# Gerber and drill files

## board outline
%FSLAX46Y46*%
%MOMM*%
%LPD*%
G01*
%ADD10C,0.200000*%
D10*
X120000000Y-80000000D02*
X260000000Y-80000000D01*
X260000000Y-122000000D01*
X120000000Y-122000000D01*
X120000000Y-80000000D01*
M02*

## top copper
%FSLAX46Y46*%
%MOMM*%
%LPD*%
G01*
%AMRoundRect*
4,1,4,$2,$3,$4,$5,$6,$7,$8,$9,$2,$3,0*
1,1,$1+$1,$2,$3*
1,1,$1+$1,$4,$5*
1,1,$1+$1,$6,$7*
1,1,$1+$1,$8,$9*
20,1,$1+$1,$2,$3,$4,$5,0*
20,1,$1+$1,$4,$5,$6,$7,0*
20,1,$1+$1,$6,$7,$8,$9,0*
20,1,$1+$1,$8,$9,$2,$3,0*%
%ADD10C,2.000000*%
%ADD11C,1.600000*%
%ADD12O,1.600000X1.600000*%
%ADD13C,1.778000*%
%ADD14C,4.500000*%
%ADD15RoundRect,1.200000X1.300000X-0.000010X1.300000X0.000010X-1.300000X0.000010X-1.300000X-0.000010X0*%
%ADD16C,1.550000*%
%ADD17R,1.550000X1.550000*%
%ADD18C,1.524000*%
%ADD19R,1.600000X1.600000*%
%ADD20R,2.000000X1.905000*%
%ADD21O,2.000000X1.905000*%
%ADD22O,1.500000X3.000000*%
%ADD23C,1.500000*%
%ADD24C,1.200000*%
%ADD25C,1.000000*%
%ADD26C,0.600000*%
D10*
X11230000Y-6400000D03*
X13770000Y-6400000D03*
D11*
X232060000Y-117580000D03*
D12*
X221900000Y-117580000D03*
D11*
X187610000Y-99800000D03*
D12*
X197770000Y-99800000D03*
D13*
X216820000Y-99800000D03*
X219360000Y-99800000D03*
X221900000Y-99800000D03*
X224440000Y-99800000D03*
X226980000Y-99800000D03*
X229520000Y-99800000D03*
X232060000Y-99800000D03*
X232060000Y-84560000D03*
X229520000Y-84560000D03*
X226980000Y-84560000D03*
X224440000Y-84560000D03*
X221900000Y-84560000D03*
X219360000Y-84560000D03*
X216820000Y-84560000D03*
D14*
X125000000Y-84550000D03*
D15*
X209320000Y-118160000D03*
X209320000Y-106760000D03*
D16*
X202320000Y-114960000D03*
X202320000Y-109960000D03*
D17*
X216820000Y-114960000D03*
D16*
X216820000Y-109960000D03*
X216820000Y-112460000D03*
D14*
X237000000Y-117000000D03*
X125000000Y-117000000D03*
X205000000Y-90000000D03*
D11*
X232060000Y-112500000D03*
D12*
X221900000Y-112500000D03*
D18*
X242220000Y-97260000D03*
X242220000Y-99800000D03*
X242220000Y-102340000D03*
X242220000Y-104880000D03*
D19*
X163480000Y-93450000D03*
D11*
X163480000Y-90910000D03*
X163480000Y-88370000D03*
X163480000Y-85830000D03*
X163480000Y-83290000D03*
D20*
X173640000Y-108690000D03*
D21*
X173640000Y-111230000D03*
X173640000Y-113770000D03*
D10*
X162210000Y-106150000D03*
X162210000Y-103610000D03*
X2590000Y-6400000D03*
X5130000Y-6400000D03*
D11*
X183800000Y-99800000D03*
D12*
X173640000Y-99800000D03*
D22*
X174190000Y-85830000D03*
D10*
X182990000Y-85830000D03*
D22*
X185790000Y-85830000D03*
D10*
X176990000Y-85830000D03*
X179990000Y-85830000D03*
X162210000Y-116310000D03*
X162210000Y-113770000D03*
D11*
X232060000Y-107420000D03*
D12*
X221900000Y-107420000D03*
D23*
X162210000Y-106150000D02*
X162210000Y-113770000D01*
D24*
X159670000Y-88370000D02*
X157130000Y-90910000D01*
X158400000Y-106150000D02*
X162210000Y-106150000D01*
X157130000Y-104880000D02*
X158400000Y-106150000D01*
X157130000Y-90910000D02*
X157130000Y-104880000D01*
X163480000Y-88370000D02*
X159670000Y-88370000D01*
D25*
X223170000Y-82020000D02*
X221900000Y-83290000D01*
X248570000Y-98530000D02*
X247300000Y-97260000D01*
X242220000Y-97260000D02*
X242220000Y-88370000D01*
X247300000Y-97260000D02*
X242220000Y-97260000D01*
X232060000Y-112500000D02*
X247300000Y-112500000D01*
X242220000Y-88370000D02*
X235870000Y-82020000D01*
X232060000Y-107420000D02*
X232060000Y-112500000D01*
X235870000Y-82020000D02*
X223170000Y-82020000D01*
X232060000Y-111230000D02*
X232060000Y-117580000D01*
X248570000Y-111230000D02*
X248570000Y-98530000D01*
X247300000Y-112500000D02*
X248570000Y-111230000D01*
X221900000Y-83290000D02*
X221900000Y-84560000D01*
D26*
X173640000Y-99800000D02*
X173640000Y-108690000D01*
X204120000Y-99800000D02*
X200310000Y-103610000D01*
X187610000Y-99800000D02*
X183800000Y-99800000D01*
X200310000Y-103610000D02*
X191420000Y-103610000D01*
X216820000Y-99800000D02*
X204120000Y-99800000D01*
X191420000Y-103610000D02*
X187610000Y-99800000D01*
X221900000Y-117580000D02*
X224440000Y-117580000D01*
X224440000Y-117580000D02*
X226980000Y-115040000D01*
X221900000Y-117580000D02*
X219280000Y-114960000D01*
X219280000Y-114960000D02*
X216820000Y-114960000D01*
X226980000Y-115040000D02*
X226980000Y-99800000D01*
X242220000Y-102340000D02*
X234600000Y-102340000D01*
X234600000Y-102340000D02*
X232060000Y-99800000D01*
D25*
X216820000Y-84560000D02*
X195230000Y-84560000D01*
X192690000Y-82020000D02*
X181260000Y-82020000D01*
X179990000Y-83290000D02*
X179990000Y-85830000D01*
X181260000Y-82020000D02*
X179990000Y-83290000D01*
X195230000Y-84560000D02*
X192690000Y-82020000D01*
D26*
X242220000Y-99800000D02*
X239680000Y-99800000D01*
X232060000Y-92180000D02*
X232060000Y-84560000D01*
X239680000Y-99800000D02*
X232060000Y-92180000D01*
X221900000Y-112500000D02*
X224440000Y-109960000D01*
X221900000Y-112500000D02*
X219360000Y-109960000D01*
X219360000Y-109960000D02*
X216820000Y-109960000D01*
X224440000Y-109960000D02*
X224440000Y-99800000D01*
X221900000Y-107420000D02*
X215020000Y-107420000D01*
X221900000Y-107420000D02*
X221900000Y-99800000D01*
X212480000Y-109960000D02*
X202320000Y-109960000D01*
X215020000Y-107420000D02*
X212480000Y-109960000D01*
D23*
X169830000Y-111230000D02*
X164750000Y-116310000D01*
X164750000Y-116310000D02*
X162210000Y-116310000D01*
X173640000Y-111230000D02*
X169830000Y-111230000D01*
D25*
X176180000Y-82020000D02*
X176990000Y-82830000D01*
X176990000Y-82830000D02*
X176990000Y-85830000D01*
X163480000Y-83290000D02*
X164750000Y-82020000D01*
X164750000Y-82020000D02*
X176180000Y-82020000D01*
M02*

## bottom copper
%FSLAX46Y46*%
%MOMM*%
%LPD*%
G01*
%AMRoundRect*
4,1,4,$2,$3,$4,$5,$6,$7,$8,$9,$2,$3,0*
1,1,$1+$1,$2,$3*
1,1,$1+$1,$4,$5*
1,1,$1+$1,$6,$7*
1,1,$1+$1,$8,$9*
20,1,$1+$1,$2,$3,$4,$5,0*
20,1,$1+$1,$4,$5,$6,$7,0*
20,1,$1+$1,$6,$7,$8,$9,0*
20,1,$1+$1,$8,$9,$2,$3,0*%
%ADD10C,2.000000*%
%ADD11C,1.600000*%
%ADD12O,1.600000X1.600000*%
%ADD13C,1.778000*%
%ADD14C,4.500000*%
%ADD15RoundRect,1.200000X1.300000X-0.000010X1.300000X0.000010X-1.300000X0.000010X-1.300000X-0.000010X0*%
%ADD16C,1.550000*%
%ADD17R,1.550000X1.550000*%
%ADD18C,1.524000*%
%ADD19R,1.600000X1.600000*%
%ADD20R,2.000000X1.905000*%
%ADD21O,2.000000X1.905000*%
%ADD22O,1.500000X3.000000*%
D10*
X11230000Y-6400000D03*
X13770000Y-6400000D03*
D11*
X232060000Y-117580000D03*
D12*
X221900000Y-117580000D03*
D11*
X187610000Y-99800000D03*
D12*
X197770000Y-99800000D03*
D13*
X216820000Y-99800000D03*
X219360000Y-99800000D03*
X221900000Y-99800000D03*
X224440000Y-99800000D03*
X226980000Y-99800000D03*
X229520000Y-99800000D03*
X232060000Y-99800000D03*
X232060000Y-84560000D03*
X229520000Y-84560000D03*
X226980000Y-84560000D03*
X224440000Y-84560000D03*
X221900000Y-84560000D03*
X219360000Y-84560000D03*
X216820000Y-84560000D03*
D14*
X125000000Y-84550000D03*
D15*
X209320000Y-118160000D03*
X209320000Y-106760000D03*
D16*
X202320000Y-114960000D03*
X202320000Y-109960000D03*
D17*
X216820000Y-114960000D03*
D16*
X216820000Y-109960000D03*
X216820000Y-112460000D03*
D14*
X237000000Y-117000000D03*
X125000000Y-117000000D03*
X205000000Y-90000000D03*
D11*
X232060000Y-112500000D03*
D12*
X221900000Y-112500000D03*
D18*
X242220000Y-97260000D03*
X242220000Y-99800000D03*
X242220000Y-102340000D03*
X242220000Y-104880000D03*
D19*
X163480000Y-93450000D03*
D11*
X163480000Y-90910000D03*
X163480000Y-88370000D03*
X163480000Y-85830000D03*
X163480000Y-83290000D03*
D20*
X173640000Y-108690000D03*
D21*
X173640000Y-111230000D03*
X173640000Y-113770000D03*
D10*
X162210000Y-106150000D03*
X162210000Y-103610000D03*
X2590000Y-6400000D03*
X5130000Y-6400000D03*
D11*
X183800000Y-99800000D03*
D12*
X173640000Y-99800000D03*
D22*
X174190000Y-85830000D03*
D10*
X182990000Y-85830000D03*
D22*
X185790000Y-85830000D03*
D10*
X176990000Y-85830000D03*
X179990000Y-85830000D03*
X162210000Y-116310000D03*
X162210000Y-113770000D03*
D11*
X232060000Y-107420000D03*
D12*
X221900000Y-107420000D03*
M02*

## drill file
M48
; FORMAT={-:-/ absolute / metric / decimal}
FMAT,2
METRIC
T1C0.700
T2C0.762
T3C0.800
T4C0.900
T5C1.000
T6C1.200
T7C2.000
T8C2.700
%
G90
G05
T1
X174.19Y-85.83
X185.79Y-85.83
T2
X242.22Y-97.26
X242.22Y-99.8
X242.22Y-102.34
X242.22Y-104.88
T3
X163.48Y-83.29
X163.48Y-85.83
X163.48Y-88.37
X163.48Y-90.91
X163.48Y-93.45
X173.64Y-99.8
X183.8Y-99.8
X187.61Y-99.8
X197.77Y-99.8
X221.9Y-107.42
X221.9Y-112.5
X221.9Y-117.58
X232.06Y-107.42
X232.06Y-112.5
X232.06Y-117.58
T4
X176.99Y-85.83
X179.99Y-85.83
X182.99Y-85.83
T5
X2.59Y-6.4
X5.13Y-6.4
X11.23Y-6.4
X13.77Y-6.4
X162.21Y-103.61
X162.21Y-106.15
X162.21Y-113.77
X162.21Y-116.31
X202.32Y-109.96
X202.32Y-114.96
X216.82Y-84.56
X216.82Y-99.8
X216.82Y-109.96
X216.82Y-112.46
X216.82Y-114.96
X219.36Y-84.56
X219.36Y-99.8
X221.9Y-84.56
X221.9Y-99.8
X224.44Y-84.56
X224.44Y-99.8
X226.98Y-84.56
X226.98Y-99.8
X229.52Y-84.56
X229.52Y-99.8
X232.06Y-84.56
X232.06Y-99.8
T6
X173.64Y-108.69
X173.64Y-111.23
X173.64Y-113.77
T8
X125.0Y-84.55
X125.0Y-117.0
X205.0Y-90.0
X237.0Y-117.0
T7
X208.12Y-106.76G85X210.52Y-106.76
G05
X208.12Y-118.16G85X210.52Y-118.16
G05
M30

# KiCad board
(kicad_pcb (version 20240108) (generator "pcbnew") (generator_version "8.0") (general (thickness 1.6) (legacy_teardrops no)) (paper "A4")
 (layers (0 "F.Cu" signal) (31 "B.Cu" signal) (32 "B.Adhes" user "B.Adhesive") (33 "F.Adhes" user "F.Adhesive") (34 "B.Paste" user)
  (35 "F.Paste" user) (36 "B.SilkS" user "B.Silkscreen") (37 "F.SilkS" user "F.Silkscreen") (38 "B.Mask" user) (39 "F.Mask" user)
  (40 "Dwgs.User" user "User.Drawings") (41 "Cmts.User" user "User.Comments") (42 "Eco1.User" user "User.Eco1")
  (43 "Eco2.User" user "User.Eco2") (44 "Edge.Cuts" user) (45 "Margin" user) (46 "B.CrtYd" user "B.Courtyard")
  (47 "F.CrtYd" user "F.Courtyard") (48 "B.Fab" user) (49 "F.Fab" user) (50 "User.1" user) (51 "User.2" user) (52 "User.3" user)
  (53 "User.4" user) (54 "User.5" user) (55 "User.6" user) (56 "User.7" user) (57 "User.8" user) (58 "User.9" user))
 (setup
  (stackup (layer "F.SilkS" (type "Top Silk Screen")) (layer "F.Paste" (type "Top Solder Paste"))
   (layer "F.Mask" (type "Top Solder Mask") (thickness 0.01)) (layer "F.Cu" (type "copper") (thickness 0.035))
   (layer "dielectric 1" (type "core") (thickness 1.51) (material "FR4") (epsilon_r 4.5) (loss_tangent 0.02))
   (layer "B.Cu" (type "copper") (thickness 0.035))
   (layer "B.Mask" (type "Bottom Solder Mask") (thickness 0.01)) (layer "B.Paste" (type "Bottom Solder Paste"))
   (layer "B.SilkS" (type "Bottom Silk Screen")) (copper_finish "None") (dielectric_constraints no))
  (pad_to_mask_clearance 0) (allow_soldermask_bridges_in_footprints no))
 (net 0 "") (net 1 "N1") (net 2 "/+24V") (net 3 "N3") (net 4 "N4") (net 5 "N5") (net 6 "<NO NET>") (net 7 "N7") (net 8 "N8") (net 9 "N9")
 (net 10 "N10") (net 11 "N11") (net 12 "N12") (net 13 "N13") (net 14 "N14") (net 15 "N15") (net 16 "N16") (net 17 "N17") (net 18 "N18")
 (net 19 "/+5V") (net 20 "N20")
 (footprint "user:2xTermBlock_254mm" (layer "F.Cu") (at 11.23 6.4)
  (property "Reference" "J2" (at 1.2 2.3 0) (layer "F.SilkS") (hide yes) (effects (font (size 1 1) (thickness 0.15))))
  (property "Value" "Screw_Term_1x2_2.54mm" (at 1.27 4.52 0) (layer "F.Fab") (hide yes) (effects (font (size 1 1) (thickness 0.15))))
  (pad "1" thru_hole circle (at 0 0) (size 2 2) (drill 1) (layers "*.Cu" "*.Mask") (remove_unused_layers no) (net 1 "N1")
   (thermal_bridge_angle 90))
  (pad "2" thru_hole circle (at 2.54 0) (size 2 2) (drill 1) (layers "*.Cu" "*.Mask") (remove_unused_layers no) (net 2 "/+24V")))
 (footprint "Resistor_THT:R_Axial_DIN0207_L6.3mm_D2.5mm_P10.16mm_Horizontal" (layer "F.Cu") (at 232.06 117.58 180)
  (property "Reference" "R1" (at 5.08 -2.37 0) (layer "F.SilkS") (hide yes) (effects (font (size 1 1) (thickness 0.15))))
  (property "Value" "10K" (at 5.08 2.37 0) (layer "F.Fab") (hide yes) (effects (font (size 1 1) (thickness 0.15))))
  (pad "1" thru_hole circle (at 0 0 180) (size 1.6 1.6) (drill 0.8) (layers "*.Cu" "*.Mask") (remove_unused_layers no) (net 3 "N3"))
  (pad "2" thru_hole oval (at 10.16 0 180) (size 1.6 1.6) (drill 0.8) (layers "*.Cu" "*.Mask") (remove_unused_layers no) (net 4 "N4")))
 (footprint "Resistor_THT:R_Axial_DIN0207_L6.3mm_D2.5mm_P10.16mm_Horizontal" (layer "F.Cu") (at 187.61 99.8)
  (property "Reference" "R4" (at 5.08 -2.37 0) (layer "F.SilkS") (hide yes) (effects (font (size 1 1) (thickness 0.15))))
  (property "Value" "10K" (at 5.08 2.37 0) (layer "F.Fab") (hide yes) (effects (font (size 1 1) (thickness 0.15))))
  (pad "1" thru_hole circle (at 0 0) (size 1.6 1.6) (drill 0.8) (layers "*.Cu" "*.Mask") (remove_unused_layers no) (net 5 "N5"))
  (pad "2" thru_hole oval (at 10.16 0) (size 1.6 1.6) (drill 0.8) (layers "*.Cu" "*.Mask") (remove_unused_layers no) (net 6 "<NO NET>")))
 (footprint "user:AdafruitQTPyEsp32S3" (layer "F.Cu") (at 216.82 99.8 90)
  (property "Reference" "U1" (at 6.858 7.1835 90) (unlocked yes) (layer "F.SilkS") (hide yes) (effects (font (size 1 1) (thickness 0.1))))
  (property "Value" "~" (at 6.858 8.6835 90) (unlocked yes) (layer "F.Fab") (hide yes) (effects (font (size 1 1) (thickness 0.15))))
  (pad "1" thru_hole circle (at 0 0 90) (size 1.778 1.778) (drill 1) (layers "*.Cu" "*.Mask") (remove_unused_layers no) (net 5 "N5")
   (solder_mask_margin 0.0508) (thermal_bridge_angle 0))
  (pad "2" thru_hole circle (at 0 2.54 90) (size 1.778 1.778) (drill 1) (layers "*.Cu" "*.Mask") (remove_unused_layers no) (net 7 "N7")
   (solder_mask_margin 0.0508) (thermal_bridge_angle 0))
  (pad "3" thru_hole circle (at 0 5.08 90) (size 1.778 1.778) (drill 1) (layers "*.Cu" "*.Mask") (remove_unused_layers no) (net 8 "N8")
   (solder_mask_margin 0.0508) (thermal_bridge_angle 0))
  (pad "4" thru_hole circle (at 0 7.62 90) (size 1.778 1.778) (drill 1) (layers "*.Cu" "*.Mask") (remove_unused_layers no) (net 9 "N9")
   (solder_mask_margin 0.0508) (thermal_bridge_angle 0))
  (pad "5" thru_hole circle (at 0 10.16 90) (size 1.778 1.778) (drill 1) (layers "*.Cu" "*.Mask") (remove_unused_layers no) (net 4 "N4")
   (solder_mask_margin 0.0508) (thermal_bridge_angle 0))
  (pad "6" thru_hole circle (at 0 12.7 90) (size 1.778 1.778) (drill 1) (layers "*.Cu" "*.Mask") (remove_unused_layers no) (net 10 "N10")
   (solder_mask_margin 0.0508) (thermal_bridge_angle 0))
  (pad "7" thru_hole circle (at 0 15.24 90) (size 1.778 1.778) (drill 1) (layers "*.Cu" "*.Mask") (remove_unused_layers no) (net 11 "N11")
   (solder_mask_margin 0.0508) (thermal_bridge_angle 0))
  (pad "8" thru_hole circle (at 15.24 15.24 270) (size 1.778 1.778) (drill 1) (layers "*.Cu" "*.Mask") (remove_unused_layers no)
   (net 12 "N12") (solder_mask_margin 0.0508) (thermal_bridge_angle 0))
  (pad "9" thru_hole circle (at 15.24 12.7 270) (size 1.778 1.778) (drill 1) (layers "*.Cu" "*.Mask") (remove_unused_layers no)
   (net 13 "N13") (solder_mask_margin 0.0508) (thermal_bridge_angle 0))
  (pad "10" thru_hole circle (at 15.24 10.16 270) (size 1.778 1.778) (drill 1) (layers "*.Cu" "*.Mask") (remove_unused_layers no)
   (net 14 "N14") (solder_mask_margin 0.0508) (thermal_bridge_angle 0))
  (pad "11" thru_hole circle (at 15.24 7.62 270) (size 1.778 1.778) (drill 1) (layers "*.Cu" "*.Mask") (remove_unused_layers no)
   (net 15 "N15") (solder_mask_margin 0.0508) (thermal_bridge_angle 0))
  (pad "12" thru_hole circle (at 15.24 5.08 270) (size 1.778 1.778) (drill 1) (layers "*.Cu" "*.Mask") (remove_unused_layers no)
   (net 3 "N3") (solder_mask_margin 0.0508) (thermal_bridge_angle 0))
  (pad "13" thru_hole circle (at 15.24 2.54 270) (size 1.778 1.778) (drill 1) (layers "*.Cu" "*.Mask") (remove_unused_layers no)
   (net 6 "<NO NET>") (solder_mask_margin 0.0508) (thermal_bridge_angle 0))
  (pad "14" thru_hole circle (at 15.24 0 270) (size 1.778 1.778) (drill 1) (layers "*.Cu" "*.Mask") (remove_unused_layers no) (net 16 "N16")
   (solder_mask_margin 0.0508) (thermal_bridge_angle 0)))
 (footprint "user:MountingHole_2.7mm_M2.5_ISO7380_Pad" (layer "F.Cu") (at 125 84.55)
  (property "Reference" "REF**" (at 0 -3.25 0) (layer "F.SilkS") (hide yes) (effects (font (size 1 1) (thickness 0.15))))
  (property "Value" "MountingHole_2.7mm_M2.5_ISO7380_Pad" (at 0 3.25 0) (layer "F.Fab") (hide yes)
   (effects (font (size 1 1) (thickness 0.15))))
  (pad "M" thru_hole circle (at 0 0) (size 4.5 4.5) (drill 2.7) (layers "*.Cu" "*.Mask") (remove_unused_layers no)))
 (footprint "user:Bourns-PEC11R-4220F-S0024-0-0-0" (layer "F.Cu") (at 209.32 112.46 90)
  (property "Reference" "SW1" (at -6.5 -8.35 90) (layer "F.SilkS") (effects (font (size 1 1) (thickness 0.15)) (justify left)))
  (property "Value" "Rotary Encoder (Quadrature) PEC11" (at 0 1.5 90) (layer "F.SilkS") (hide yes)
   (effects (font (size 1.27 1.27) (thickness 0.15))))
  (pad "" thru_hole roundrect (at -5.7 0 90) (size 2.4 5) (drill oval 2 4.4) (layers "*.Cu" "*.Mask") (remove_unused_layers no)
   (roundrect_rratio 0.5))
  (pad "" thru_hole roundrect (at 5.7 0 90) (size 2.4 5) (drill oval 2 4.4) (layers "*.Cu" "*.Mask") (remove_unused_layers no)
   (roundrect_rratio 0.5))
  (pad "1" thru_hole circle (at -2.5 -7 90) (size 1.55 1.55) (drill 1) (layers "*.Cu" "*.Mask") (remove_unused_layers no) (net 6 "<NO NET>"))
  (pad "2" thru_hole circle (at 2.5 -7 90) (size 1.55 1.55) (drill 1) (layers "*.Cu" "*.Mask") (remove_unused_layers no) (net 8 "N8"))
  (pad "A" thru_hole rect (at -2.5 7.5 90) (size 1.55 1.55) (drill 1) (layers "*.Cu" "*.Mask") (remove_unused_layers no) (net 4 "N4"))
  (pad "B" thru_hole circle (at 2.5 7.5 90) (size 1.55 1.55) (drill 1) (layers "*.Cu" "*.Mask") (remove_unused_layers no) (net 9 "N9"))
  (pad "C" thru_hole circle (at 0 7.5 90) (size 1.55 1.55) (drill 1) (layers "*.Cu" "*.Mask") (remove_unused_layers no) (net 6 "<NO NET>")))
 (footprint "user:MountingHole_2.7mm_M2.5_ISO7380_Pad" (layer "F.Cu") (at 237 117)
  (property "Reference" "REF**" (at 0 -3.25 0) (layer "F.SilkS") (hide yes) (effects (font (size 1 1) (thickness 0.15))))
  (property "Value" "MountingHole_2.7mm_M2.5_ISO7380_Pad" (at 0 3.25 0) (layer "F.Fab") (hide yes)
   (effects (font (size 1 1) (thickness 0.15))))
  (pad "M" thru_hole circle (at 0 0) (size 4.5 4.5) (drill 2.7) (layers "*.Cu" "*.Mask") (remove_unused_layers no)))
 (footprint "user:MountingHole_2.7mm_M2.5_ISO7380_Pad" (layer "F.Cu") (at 125 117)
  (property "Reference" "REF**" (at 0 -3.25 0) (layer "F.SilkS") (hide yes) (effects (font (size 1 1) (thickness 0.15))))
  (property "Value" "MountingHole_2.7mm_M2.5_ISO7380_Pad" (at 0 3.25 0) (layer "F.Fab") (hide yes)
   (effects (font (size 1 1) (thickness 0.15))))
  (pad "M" thru_hole circle (at 0 0) (size 4.5 4.5) (drill 2.7) (layers "*.Cu" "*.Mask") (remove_unused_layers no)))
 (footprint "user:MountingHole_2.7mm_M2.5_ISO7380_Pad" (layer "F.Cu") (at 205 90)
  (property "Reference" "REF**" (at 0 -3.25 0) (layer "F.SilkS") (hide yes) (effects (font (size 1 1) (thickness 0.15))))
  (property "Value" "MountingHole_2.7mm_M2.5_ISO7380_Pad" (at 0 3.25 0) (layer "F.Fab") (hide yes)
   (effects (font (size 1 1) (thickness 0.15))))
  (pad "M" thru_hole circle (at 0 0) (size 4.5 4.5) (drill 2.7) (layers "*.Cu" "*.Mask") (remove_unused_layers no)))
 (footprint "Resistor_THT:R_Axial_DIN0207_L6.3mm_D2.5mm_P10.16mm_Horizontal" (layer "F.Cu") (at 232.06 112.5 180)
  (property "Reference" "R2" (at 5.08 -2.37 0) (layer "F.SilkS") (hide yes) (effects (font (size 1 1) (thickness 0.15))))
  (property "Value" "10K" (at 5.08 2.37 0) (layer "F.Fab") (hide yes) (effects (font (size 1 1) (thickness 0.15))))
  (pad "1" thru_hole circle (at 0 0 180) (size 1.6 1.6) (drill 0.8) (layers "*.Cu" "*.Mask") (remove_unused_layers no) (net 3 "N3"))
  (pad "2" thru_hole oval (at 10.16 0 180) (size 1.6 1.6) (drill 0.8) (layers "*.Cu" "*.Mask") (remove_unused_layers no) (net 9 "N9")))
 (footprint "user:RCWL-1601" (layer "F.Cu") (at 242.22 97.26 -90)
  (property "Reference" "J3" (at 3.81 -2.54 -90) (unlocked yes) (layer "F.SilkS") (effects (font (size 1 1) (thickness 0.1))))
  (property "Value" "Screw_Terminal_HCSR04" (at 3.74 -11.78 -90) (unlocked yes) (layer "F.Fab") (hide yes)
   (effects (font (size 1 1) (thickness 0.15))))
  (pad "1" thru_hole circle (at 0 0 270) (size 1.524 1.524) (drill 0.762) (layers "*.Cu" "*.Mask") (remove_unused_layers no) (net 3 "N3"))
  (pad "2" thru_hole circle (at 2.54 0 270) (size 1.524 1.524) (drill 0.762) (layers "*.Cu" "*.Mask") (remove_unused_layers no)
   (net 12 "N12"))
  (pad "3" thru_hole circle (at 5.08 0 270) (size 1.524 1.524) (drill 0.762) (layers "*.Cu" "*.Mask") (remove_unused_layers no)
   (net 11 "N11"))
  (pad "4" thru_hole circle (at 7.62 0 270) (size 1.524 1.524) (drill 0.762) (layers "*.Cu" "*.Mask") (remove_unused_layers no)
   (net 6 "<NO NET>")))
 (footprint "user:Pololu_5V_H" (layer "F.Cu") (at 163.48 88.37 90)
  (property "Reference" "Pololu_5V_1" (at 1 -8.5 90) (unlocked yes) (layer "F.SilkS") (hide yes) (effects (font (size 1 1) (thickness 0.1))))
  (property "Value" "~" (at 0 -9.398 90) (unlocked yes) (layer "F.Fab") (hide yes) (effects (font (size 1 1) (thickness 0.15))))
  (pad "1" thru_hole rect (at -5.08 0 90) (size 1.6 1.6) (drill 0.8) (layers "*.Cu" "*.Mask") (remove_unused_layers no) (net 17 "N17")
   (thermal_bridge_angle 45))
  (pad "2" thru_hole circle (at -2.54 0 90) (size 1.6 1.6) (drill 0.8) (layers "*.Cu" "*.Mask") (remove_unused_layers no) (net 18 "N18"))
  (pad "3" thru_hole circle (at 0 0 90) (size 1.6 1.6) (drill 0.8) (layers "*.Cu" "*.Mask") (remove_unused_layers no) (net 2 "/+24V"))
  (pad "4" thru_hole circle (at 2.54 0 90) (size 1.6 1.6) (drill 0.8) (layers "*.Cu" "*.Mask") (remove_unused_layers no) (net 6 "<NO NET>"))
  (pad "5" thru_hole circle (at 5.08 0 90) (size 1.6 1.6) (drill 0.8) (layers "*.Cu" "*.Mask") (remove_unused_layers no) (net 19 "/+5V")))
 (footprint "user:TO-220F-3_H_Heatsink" (layer "F.Cu") (at 173.64 108.69 -90)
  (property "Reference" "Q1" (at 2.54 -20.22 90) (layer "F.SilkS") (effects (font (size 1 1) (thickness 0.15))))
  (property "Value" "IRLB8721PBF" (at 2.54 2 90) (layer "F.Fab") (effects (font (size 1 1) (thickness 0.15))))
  (pad "1" thru_hole rect (at 0 0 270) (size 1.905 2) (drill 1.2) (layers "*.Cu" "*.Mask") (remove_unused_layers no) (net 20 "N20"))
  (pad "2" thru_hole oval (at 2.54 0 270) (size 1.905 2) (drill 1.2) (layers "*.Cu" "*.Mask") (remove_unused_layers no) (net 1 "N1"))
  (pad "3" thru_hole oval (at 5.08 0 270) (size 1.905 2) (drill 1.2) (layers "*.Cu" "*.Mask") (remove_unused_layers no) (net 6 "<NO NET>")))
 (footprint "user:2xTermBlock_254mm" (layer "F.Cu") (at 162.21 106.15 90)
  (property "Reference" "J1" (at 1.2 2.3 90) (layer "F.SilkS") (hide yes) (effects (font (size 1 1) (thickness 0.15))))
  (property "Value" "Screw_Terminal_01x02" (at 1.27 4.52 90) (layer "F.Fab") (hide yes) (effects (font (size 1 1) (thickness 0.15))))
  (pad "1" thru_hole circle (at 0 0 90) (size 2 2) (drill 1) (layers "*.Cu" "*.Mask") (remove_unused_layers no) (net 2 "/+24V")
   (thermal_bridge_angle 90))
  (pad "2" thru_hole circle (at 2.54 0 90) (size 2 2) (drill 1) (layers "*.Cu" "*.Mask") (remove_unused_layers no) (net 6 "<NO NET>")))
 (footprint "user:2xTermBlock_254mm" (layer "F.Cu") (at 2.59 6.4)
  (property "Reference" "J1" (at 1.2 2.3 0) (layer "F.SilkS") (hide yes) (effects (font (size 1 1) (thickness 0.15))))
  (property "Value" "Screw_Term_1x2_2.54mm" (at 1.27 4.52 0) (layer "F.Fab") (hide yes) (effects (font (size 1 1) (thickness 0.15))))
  (pad "1" thru_hole circle (at 0 0) (size 2 2) (drill 1) (layers "*.Cu" "*.Mask") (remove_unused_layers no) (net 2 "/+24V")
   (thermal_bridge_angle 90))
  (pad "2" thru_hole circle (at 2.54 0) (size 2 2) (drill 1) (layers "*.Cu" "*.Mask") (remove_unused_layers no) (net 6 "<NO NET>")))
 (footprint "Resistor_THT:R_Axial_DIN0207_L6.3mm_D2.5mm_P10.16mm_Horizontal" (layer "F.Cu") (at 183.8 99.8 180)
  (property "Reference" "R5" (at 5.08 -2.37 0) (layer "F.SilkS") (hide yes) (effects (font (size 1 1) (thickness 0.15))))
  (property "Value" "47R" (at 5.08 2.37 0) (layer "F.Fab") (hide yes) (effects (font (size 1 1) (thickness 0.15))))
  (pad "1" thru_hole circle (at 0 0 180) (size 1.6 1.6) (drill 0.8) (layers "*.Cu" "*.Mask") (remove_unused_layers no) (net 5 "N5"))
  (pad "2" thru_hole oval (at 10.16 0 180) (size 1.6 1.6) (drill 0.8) (layers "*.Cu" "*.Mask") (remove_unused_layers no) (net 20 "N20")))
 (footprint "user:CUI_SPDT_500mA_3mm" (layer "F.Cu") (at 179.99 85.83)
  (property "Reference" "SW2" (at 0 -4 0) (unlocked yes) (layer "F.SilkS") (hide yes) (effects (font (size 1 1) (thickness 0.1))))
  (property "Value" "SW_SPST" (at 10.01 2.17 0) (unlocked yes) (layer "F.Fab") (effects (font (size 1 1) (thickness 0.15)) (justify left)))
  (pad "" thru_hole oval (at -5.8 0) (size 1.5 3) (drill 0.7 1.5) (layers "*.Cu" "*.Mask") (remove_unused_layers no)
   (thermal_bridge_angle 45))
  (pad "" thru_hole circle (at 3 0) (size 2 2) (drill 0.9) (layers "*.Cu" "*.Mask") (remove_unused_layers no))
  (pad "" thru_hole oval (at 5.8 0) (size 1.5 3) (drill 0.7 1.5) (layers "*.Cu" "*.Mask") (remove_unused_layers no)
   (thermal_bridge_angle 45))
  (pad "1" thru_hole circle (at -3 0) (size 2 2) (drill 0.9) (layers "*.Cu" "*.Mask") (remove_unused_layers no) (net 19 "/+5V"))
  (pad "2" thru_hole circle (at 0 0) (size 2 2) (drill 0.9) (layers "*.Cu" "*.Mask") (remove_unused_layers no) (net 16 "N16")))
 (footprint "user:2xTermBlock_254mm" (layer "F.Cu") (at 162.21 116.31 90)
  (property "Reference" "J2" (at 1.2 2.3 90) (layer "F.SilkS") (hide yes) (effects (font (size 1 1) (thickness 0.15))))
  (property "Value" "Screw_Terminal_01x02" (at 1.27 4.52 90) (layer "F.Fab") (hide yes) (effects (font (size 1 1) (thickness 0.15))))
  (pad "1" thru_hole circle (at 0 0 90) (size 2 2) (drill 1) (layers "*.Cu" "*.Mask") (remove_unused_layers no) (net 1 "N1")
   (thermal_bridge_angle 90))
  (pad "2" thru_hole circle (at 2.54 0 90) (size 2 2) (drill 1) (layers "*.Cu" "*.Mask") (remove_unused_layers no) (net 2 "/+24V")))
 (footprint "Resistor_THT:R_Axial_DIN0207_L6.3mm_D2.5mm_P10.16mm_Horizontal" (layer "F.Cu") (at 232.06 107.42 180)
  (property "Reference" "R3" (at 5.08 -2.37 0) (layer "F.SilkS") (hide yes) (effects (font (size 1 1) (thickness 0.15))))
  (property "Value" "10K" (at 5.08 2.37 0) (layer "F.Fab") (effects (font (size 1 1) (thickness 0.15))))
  (pad "1" thru_hole circle (at 0 0 180) (size 1.6 1.6) (drill 0.8) (layers "*.Cu" "*.Mask") (remove_unused_layers no) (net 3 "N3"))
  (pad "2" thru_hole oval (at 10.16 0 180) (size 1.6 1.6) (drill 0.8) (layers "*.Cu" "*.Mask") (remove_unused_layers no) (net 8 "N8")))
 (gr_rect (start 120 80) (end 260 122) (stroke (width 0.2) (type default)) (fill none) (layer "Edge.Cuts"))
 (segment (start 162.21 106.15) (end 162.21 113.77) (width 1.5) (layer "F.Cu") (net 2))
 (segment (start 159.67 88.37) (end 157.13 90.91) (width 1.2) (layer "F.Cu") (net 2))
 (segment (start 158.4 106.15) (end 162.21 106.15) (width 1.2) (layer "F.Cu") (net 2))
 (segment (start 157.13 104.88) (end 158.4 106.15) (width 1.2) (layer "F.Cu") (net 2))
 (segment (start 157.13 90.91) (end 157.13 104.88) (width 1.2) (layer "F.Cu") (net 2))
 (segment (start 163.48 88.37) (end 159.67 88.37) (width 1.2) (layer "F.Cu") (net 2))
 (segment (start 223.17 82.02) (end 221.9 83.29) (width 1) (layer "F.Cu") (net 3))
 (segment (start 248.57 98.53) (end 247.3 97.26) (width 1) (layer "F.Cu") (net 3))
 (segment (start 242.22 97.26) (end 242.22 88.37) (width 1) (layer "F.Cu") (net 3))
 (segment (start 247.3 97.26) (end 242.22 97.26) (width 1) (layer "F.Cu") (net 3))
 (segment (start 232.06 112.5) (end 247.3 112.5) (width 1) (layer "F.Cu") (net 3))
 (segment (start 242.22 88.37) (end 235.87 82.02) (width 1) (layer "F.Cu") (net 3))
 (segment (start 232.06 107.42) (end 232.06 112.5) (width 1) (layer "F.Cu") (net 3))
 (segment (start 235.87 82.02) (end 223.17 82.02) (width 1) (layer "F.Cu") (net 3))
 (segment (start 232.06 111.23) (end 232.06 117.58) (width 1) (layer "F.Cu") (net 3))
 (segment (start 248.57 111.23) (end 248.57 98.53) (width 1) (layer "F.Cu") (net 3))
 (segment (start 247.3 112.5) (end 248.57 111.23) (width 1) (layer "F.Cu") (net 3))
 (segment (start 221.9 83.29) (end 221.9 84.56) (width 1) (layer "F.Cu") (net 3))
 (segment (start 173.64 99.8) (end 173.64 108.69) (width 0.6) (layer "F.Cu") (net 20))
 (segment (start 204.12 99.8) (end 200.31 103.61) (width 0.6) (layer "F.Cu") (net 5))
 (segment (start 187.61 99.8) (end 183.8 99.8) (width 0.6) (layer "F.Cu") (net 5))
 (segment (start 200.31 103.61) (end 191.42 103.61) (width 0.6) (layer "F.Cu") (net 5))
 (segment (start 216.82 99.8) (end 204.12 99.8) (width 0.6) (layer "F.Cu") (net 5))
 (segment (start 191.42 103.61) (end 187.61 99.8) (width 0.6) (layer "F.Cu") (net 5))
 (segment (start 221.9 117.58) (end 224.44 117.58) (width 0.6) (layer "F.Cu") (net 4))
 (segment (start 224.44 117.58) (end 226.98 115.04) (width 0.6) (layer "F.Cu") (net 4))
 (segment (start 221.9 117.58) (end 219.28 114.96) (width 0.6) (layer "F.Cu") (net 4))
 (segment (start 219.28 114.96) (end 216.82 114.96) (width 0.6) (layer "F.Cu") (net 4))
 (segment (start 226.98 115.04) (end 226.98 99.8) (width 0.6) (layer "F.Cu") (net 4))
 (segment (start 242.22 102.34) (end 234.6 102.34) (width 0.6) (layer "F.Cu") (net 11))
 (segment (start 234.6 102.34) (end 232.06 99.8) (width 0.6) (layer "F.Cu") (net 11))
 (segment (start 216.82 84.56) (end 195.23 84.56) (width 1) (layer "F.Cu") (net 16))
 (segment (start 192.69 82.02) (end 181.26 82.02) (width 1) (layer "F.Cu") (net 16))
 (segment (start 179.99 83.29) (end 179.99 85.83) (width 1) (layer "F.Cu") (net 16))
 (segment (start 181.26 82.02) (end 179.99 83.29) (width 1) (layer "F.Cu") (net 16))
 (segment (start 195.23 84.56) (end 192.69 82.02) (width 1) (layer "F.Cu") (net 16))
 (segment (start 242.22 99.8) (end 239.68 99.8) (width 0.6) (layer "F.Cu") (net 12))
 (segment (start 232.06 92.18) (end 232.06 84.56) (width 0.6) (layer "F.Cu") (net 12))
 (segment (start 239.68 99.8) (end 232.06 92.18) (width 0.6) (layer "F.Cu") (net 12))
 (segment (start 221.9 112.5) (end 224.44 109.96) (width 0.6) (layer "F.Cu") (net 9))
 (segment (start 221.9 112.5) (end 219.36 109.96) (width 0.6) (layer "F.Cu") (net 9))
 (segment (start 219.36 109.96) (end 216.82 109.96) (width 0.6) (layer "F.Cu") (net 9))
 (segment (start 224.44 109.96) (end 224.44 99.8) (width 0.6) (layer "F.Cu") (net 9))
 (segment (start 221.9 107.42) (end 215.02 107.42) (width 0.6) (layer "F.Cu") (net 8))
 (segment (start 221.9 107.42) (end 221.9 99.8) (width 0.6) (layer "F.Cu") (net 8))
 (segment (start 212.48 109.96) (end 202.32 109.96) (width 0.6) (layer "F.Cu") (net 8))
 (segment (start 215.02 107.42) (end 212.48 109.96) (width 0.6) (layer "F.Cu") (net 8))
 (segment (start 169.83 111.23) (end 164.75 116.31) (width 1.5) (layer "F.Cu") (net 1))
 (segment (start 164.75 116.31) (end 162.21 116.31) (width 1.5) (layer "F.Cu") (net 1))
 (segment (start 173.64 111.23) (end 169.83 111.23) (width 1.5) (layer "F.Cu") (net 1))
 (segment (start 176.18 82.02) (end 176.99 82.83) (width 1) (layer "F.Cu") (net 19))
 (segment (start 176.99 82.83) (end 176.99 85.83) (width 1) (layer "F.Cu") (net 19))
 (segment (start 163.48 83.29) (end 164.75 82.02) (width 1) (layer "F.Cu") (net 19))
 (segment (start 164.75 82.02) (end 176.18 82.02) (width 1) (layer "F.Cu") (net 19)))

